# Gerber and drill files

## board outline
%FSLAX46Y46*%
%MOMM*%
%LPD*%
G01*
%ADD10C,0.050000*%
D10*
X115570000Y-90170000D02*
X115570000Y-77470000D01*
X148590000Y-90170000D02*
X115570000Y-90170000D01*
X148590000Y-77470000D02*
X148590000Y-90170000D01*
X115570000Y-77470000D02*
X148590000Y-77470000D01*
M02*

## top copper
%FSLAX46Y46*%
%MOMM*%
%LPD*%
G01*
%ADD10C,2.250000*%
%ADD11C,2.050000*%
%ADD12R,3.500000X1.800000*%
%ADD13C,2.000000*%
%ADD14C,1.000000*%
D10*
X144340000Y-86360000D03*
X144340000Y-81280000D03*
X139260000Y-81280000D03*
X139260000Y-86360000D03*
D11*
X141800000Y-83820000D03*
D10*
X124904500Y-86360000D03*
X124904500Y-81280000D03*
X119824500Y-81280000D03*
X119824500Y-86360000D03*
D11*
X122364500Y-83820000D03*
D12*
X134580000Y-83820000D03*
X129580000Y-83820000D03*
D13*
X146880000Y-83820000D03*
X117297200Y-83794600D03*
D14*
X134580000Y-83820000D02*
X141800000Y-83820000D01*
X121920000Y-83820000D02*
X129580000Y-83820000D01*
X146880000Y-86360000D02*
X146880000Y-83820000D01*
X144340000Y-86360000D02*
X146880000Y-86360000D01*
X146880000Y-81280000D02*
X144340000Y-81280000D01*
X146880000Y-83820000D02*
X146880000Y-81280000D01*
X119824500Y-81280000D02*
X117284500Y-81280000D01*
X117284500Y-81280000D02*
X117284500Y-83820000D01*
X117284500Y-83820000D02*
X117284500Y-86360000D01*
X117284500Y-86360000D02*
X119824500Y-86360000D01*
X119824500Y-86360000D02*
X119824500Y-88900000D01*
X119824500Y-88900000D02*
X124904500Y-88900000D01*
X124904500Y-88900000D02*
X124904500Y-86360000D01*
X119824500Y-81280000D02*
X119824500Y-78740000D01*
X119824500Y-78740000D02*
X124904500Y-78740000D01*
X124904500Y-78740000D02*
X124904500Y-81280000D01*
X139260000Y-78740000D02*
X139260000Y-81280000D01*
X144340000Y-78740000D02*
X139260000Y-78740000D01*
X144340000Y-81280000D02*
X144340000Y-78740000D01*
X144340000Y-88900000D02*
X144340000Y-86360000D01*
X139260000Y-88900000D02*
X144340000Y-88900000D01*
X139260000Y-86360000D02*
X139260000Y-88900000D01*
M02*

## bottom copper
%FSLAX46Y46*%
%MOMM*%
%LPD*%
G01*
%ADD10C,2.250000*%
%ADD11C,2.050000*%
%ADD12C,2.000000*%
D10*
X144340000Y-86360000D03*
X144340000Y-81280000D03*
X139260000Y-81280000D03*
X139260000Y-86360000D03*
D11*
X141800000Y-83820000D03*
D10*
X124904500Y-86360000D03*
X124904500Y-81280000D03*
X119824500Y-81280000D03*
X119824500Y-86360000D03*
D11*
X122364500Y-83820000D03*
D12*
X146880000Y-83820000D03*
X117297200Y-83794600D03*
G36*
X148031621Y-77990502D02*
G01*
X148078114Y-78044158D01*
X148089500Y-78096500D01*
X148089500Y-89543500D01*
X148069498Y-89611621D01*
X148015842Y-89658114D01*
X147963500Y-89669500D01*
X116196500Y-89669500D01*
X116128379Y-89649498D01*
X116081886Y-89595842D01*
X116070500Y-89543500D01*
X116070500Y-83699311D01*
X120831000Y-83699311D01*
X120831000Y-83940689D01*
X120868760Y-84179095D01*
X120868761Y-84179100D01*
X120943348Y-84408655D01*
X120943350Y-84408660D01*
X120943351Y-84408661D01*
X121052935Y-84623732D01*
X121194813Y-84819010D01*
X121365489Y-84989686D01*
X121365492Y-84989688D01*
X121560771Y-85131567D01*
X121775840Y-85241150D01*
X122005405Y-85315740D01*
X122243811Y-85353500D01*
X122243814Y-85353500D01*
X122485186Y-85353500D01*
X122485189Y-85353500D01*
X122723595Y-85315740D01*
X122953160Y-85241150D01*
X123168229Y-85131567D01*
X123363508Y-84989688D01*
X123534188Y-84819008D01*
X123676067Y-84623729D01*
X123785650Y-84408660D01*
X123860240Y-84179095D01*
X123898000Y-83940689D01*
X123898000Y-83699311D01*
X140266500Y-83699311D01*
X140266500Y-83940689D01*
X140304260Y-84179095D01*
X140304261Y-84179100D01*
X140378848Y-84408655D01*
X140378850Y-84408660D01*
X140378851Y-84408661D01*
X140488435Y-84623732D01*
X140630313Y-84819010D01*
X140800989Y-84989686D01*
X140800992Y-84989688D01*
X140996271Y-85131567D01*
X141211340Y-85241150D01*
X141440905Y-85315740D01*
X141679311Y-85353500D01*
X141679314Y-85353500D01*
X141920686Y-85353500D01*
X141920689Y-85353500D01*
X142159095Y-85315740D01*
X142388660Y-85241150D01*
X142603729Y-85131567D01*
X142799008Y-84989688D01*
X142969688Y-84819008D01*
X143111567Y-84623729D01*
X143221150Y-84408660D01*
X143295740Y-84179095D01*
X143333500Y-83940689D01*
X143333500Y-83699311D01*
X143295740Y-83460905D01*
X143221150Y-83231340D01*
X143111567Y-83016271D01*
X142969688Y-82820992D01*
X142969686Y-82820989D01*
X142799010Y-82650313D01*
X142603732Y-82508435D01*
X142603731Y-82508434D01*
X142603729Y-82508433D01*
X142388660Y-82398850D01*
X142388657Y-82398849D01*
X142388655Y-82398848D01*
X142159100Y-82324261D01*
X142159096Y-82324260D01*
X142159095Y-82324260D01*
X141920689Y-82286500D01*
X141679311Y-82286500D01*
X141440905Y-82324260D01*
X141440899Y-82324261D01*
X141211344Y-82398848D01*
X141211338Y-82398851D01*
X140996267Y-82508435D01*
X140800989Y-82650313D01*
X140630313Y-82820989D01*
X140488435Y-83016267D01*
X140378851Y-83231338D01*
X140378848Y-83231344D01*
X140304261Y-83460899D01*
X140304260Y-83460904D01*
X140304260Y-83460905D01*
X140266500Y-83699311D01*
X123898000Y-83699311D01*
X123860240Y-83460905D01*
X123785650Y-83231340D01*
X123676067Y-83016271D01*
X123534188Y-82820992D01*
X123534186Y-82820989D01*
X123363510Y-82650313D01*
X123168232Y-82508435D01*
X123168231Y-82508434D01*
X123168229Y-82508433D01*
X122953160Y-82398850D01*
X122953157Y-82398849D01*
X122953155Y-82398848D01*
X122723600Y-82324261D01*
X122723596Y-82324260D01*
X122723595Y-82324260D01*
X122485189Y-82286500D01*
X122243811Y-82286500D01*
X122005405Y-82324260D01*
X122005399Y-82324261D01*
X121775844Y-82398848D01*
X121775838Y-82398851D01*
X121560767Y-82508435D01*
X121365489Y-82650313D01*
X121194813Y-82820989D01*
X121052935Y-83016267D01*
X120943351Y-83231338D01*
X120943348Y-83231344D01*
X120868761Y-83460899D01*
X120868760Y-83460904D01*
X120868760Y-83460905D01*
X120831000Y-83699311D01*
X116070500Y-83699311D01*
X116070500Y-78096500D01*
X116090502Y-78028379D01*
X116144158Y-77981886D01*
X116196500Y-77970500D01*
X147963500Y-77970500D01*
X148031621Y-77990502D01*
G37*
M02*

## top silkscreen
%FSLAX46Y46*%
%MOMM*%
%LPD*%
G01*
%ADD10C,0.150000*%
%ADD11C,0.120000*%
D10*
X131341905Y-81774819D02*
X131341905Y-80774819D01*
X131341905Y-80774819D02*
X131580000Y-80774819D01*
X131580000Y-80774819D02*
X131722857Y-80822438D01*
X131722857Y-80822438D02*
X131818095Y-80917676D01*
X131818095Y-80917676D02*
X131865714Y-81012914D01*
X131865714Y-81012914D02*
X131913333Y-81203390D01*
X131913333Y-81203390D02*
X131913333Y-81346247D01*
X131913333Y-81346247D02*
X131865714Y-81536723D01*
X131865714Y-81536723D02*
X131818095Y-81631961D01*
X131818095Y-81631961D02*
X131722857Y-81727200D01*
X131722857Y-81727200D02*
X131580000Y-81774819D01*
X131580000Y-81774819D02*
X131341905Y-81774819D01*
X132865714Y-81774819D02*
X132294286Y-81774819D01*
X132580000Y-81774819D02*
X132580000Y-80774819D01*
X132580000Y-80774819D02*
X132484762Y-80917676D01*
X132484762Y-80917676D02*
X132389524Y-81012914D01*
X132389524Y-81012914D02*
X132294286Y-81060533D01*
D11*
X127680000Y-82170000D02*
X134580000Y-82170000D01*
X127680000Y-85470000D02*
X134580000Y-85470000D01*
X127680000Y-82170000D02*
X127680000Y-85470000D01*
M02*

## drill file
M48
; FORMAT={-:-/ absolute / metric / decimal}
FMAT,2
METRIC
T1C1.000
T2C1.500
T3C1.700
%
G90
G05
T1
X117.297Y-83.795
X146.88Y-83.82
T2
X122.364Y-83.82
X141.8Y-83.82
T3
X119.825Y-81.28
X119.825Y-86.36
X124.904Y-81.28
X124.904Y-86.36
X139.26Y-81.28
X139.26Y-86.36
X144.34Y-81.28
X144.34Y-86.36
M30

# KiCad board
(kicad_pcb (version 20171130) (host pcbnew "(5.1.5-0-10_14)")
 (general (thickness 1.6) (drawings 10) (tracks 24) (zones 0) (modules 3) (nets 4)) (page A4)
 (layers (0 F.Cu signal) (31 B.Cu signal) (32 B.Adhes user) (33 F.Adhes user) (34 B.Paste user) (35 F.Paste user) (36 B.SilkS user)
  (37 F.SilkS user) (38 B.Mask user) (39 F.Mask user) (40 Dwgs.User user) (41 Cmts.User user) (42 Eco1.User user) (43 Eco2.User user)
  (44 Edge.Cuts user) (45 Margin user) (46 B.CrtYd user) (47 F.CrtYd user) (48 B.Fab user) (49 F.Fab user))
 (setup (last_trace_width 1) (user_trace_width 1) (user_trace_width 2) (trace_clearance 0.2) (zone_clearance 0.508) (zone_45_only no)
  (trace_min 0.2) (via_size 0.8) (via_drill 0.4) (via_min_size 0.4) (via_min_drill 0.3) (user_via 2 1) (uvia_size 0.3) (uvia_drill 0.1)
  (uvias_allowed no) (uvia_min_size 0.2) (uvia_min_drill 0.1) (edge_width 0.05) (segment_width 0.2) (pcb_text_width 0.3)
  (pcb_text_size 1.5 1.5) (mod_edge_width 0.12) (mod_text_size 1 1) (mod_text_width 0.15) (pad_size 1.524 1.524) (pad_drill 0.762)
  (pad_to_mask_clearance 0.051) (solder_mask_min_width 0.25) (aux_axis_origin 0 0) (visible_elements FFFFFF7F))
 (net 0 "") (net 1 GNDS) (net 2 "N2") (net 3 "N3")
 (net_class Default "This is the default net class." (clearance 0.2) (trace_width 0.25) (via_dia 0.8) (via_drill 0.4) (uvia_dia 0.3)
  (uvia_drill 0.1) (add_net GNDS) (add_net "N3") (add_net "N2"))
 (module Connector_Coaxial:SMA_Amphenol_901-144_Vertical (layer B.Cu) (at 141.8 83.82 180)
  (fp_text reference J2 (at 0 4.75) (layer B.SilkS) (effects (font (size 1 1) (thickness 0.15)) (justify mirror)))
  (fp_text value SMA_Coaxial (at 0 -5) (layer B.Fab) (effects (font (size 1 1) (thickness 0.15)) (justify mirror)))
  (pad 2 thru_hole circle (at -2.54 -2.54 180) (size 2.25 2.25) (drill 1.7) (layers *.Cu *.Mask) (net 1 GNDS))
  (pad 2 thru_hole circle (at -2.54 2.54 180) (size 2.25 2.25) (drill 1.7) (layers *.Cu *.Mask) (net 1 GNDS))
  (pad 2 thru_hole circle (at 2.54 2.54 180) (size 2.25 2.25) (drill 1.7) (layers *.Cu *.Mask) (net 1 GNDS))
  (pad 2 thru_hole circle (at 2.54 -2.54 180) (size 2.25 2.25) (drill 1.7) (layers *.Cu *.Mask) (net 1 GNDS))
  (pad 1 thru_hole circle (at 0 0 180) (size 2.05 2.05) (drill 1.5) (layers *.Cu *.Mask) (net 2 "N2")))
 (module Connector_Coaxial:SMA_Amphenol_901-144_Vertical (layer B.Cu) (at 122.3645 83.82 180)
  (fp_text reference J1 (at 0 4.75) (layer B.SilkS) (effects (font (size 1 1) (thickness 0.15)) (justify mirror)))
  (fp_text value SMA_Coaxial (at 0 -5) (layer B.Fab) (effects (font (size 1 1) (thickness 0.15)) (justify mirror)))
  (pad 2 thru_hole circle (at -2.54 -2.54 180) (size 2.25 2.25) (drill 1.7) (layers *.Cu *.Mask) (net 1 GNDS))
  (pad 2 thru_hole circle (at -2.54 2.54 180) (size 2.25 2.25) (drill 1.7) (layers *.Cu *.Mask) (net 1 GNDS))
  (pad 2 thru_hole circle (at 2.54 2.54 180) (size 2.25 2.25) (drill 1.7) (layers *.Cu *.Mask) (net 1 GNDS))
  (pad 2 thru_hole circle (at 2.54 -2.54 180) (size 2.25 2.25) (drill 1.7) (layers *.Cu *.Mask) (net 1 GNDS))
  (pad 1 thru_hole circle (at 0 0 180) (size 2.05 2.05) (drill 1.5) (layers *.Cu *.Mask) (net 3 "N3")))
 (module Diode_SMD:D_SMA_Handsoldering (layer F.Cu) (at 132.08 83.82)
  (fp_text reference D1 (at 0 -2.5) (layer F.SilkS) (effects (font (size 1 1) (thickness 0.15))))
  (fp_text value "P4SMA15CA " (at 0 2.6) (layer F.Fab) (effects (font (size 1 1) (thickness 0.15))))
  (fp_line (start -4.4 -1.65) (end 2.5 -1.65) (layer F.SilkS) (width 0.12))
  (fp_line (start -4.4 1.65) (end 2.5 1.65) (layer F.SilkS) (width 0.12))
  (fp_line (start -4.4 -1.65) (end -4.4 1.65) (layer F.SilkS) (width 0.12))
  (pad 2 smd rect (at 2.5 0) (size 3.5 1.8) (layers F.Cu F.Paste F.Mask) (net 2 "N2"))
  (pad 1 smd rect (at -2.5 0) (size 3.5 1.8) (layers F.Cu F.Paste F.Mask) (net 3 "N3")))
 (gr_line (start 115.57 90.17) (end 115.57 77.47) (layer Edge.Cuts) (width 0.05))
 (gr_line (start 148.59 90.17) (end 115.57 90.17) (layer Edge.Cuts) (width 0.05))
 (gr_line (start 148.59 77.47) (end 148.59 90.17) (layer Edge.Cuts) (width 0.05))
 (gr_line (start 115.57 77.47) (end 148.59 77.47) (layer Edge.Cuts) (width 0.05))
 (segment (start 134.58 83.82) (end 141.8 83.82) (width 1) (layer F.Cu) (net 2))
 (segment (start 121.92 83.82) (end 129.58 83.82) (width 1) (layer F.Cu) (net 3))
 (via (at 146.88 83.82) (size 2) (drill 1) (layers F.Cu B.Cu) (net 1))
 (segment (start 146.88 86.36) (end 146.88 83.82) (width 1) (layer F.Cu) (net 1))
 (segment (start 144.34 86.36) (end 146.88 86.36) (width 1) (layer F.Cu) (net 1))
 (segment (start 146.88 81.28) (end 144.34 81.28) (width 1) (layer F.Cu) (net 1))
 (segment (start 146.88 83.82) (end 146.88 81.28) (width 1) (layer F.Cu) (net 1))
 (segment (start 119.8245 81.28) (end 117.2845 81.28) (width 1) (layer F.Cu) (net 1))
 (segment (start 117.2845 81.28) (end 117.2845 83.82) (width 1) (layer F.Cu) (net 1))
 (via (at 117.2972 83.7946) (size 2) (drill 1) (layers F.Cu B.Cu) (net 1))
 (segment (start 117.2845 83.82) (end 117.2845 86.36) (width 1) (layer F.Cu) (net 1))
 (segment (start 117.2845 86.36) (end 119.8245 86.36) (width 1) (layer F.Cu) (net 1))
 (segment (start 119.8245 86.36) (end 119.8245 88.9) (width 1) (layer F.Cu) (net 1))
 (segment (start 119.8245 88.9) (end 124.9045 88.9) (width 1) (layer F.Cu) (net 1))
 (segment (start 124.9045 88.9) (end 124.9045 86.36) (width 1) (layer F.Cu) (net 1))
 (segment (start 119.8245 81.28) (end 119.8245 78.74) (width 1) (layer F.Cu) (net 1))
 (segment (start 119.8245 78.74) (end 124.9045 78.74) (width 1) (layer F.Cu) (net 1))
 (segment (start 124.9045 78.74) (end 124.9045 81.28) (width 1) (layer F.Cu) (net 1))
 (segment (start 139.26 78.74) (end 139.26 81.28) (width 1) (layer F.Cu) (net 1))
 (segment (start 144.34 78.74) (end 139.26 78.74) (width 1) (layer F.Cu) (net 1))
 (segment (start 144.34 81.28) (end 144.34 78.74) (width 1) (layer F.Cu) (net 1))
 (segment (start 144.34 88.9) (end 144.34 86.36) (width 1) (layer F.Cu) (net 1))
 (segment (start 139.26 88.9) (end 144.34 88.9) (width 1) (layer F.Cu) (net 1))
 (segment (start 139.26 86.36) (end 139.26 88.9) (width 1) (layer F.Cu) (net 1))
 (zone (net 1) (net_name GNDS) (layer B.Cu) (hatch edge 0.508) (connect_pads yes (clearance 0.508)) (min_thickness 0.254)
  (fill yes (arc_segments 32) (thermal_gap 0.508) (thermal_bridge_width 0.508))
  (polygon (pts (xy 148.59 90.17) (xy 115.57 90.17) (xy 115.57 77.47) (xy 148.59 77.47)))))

